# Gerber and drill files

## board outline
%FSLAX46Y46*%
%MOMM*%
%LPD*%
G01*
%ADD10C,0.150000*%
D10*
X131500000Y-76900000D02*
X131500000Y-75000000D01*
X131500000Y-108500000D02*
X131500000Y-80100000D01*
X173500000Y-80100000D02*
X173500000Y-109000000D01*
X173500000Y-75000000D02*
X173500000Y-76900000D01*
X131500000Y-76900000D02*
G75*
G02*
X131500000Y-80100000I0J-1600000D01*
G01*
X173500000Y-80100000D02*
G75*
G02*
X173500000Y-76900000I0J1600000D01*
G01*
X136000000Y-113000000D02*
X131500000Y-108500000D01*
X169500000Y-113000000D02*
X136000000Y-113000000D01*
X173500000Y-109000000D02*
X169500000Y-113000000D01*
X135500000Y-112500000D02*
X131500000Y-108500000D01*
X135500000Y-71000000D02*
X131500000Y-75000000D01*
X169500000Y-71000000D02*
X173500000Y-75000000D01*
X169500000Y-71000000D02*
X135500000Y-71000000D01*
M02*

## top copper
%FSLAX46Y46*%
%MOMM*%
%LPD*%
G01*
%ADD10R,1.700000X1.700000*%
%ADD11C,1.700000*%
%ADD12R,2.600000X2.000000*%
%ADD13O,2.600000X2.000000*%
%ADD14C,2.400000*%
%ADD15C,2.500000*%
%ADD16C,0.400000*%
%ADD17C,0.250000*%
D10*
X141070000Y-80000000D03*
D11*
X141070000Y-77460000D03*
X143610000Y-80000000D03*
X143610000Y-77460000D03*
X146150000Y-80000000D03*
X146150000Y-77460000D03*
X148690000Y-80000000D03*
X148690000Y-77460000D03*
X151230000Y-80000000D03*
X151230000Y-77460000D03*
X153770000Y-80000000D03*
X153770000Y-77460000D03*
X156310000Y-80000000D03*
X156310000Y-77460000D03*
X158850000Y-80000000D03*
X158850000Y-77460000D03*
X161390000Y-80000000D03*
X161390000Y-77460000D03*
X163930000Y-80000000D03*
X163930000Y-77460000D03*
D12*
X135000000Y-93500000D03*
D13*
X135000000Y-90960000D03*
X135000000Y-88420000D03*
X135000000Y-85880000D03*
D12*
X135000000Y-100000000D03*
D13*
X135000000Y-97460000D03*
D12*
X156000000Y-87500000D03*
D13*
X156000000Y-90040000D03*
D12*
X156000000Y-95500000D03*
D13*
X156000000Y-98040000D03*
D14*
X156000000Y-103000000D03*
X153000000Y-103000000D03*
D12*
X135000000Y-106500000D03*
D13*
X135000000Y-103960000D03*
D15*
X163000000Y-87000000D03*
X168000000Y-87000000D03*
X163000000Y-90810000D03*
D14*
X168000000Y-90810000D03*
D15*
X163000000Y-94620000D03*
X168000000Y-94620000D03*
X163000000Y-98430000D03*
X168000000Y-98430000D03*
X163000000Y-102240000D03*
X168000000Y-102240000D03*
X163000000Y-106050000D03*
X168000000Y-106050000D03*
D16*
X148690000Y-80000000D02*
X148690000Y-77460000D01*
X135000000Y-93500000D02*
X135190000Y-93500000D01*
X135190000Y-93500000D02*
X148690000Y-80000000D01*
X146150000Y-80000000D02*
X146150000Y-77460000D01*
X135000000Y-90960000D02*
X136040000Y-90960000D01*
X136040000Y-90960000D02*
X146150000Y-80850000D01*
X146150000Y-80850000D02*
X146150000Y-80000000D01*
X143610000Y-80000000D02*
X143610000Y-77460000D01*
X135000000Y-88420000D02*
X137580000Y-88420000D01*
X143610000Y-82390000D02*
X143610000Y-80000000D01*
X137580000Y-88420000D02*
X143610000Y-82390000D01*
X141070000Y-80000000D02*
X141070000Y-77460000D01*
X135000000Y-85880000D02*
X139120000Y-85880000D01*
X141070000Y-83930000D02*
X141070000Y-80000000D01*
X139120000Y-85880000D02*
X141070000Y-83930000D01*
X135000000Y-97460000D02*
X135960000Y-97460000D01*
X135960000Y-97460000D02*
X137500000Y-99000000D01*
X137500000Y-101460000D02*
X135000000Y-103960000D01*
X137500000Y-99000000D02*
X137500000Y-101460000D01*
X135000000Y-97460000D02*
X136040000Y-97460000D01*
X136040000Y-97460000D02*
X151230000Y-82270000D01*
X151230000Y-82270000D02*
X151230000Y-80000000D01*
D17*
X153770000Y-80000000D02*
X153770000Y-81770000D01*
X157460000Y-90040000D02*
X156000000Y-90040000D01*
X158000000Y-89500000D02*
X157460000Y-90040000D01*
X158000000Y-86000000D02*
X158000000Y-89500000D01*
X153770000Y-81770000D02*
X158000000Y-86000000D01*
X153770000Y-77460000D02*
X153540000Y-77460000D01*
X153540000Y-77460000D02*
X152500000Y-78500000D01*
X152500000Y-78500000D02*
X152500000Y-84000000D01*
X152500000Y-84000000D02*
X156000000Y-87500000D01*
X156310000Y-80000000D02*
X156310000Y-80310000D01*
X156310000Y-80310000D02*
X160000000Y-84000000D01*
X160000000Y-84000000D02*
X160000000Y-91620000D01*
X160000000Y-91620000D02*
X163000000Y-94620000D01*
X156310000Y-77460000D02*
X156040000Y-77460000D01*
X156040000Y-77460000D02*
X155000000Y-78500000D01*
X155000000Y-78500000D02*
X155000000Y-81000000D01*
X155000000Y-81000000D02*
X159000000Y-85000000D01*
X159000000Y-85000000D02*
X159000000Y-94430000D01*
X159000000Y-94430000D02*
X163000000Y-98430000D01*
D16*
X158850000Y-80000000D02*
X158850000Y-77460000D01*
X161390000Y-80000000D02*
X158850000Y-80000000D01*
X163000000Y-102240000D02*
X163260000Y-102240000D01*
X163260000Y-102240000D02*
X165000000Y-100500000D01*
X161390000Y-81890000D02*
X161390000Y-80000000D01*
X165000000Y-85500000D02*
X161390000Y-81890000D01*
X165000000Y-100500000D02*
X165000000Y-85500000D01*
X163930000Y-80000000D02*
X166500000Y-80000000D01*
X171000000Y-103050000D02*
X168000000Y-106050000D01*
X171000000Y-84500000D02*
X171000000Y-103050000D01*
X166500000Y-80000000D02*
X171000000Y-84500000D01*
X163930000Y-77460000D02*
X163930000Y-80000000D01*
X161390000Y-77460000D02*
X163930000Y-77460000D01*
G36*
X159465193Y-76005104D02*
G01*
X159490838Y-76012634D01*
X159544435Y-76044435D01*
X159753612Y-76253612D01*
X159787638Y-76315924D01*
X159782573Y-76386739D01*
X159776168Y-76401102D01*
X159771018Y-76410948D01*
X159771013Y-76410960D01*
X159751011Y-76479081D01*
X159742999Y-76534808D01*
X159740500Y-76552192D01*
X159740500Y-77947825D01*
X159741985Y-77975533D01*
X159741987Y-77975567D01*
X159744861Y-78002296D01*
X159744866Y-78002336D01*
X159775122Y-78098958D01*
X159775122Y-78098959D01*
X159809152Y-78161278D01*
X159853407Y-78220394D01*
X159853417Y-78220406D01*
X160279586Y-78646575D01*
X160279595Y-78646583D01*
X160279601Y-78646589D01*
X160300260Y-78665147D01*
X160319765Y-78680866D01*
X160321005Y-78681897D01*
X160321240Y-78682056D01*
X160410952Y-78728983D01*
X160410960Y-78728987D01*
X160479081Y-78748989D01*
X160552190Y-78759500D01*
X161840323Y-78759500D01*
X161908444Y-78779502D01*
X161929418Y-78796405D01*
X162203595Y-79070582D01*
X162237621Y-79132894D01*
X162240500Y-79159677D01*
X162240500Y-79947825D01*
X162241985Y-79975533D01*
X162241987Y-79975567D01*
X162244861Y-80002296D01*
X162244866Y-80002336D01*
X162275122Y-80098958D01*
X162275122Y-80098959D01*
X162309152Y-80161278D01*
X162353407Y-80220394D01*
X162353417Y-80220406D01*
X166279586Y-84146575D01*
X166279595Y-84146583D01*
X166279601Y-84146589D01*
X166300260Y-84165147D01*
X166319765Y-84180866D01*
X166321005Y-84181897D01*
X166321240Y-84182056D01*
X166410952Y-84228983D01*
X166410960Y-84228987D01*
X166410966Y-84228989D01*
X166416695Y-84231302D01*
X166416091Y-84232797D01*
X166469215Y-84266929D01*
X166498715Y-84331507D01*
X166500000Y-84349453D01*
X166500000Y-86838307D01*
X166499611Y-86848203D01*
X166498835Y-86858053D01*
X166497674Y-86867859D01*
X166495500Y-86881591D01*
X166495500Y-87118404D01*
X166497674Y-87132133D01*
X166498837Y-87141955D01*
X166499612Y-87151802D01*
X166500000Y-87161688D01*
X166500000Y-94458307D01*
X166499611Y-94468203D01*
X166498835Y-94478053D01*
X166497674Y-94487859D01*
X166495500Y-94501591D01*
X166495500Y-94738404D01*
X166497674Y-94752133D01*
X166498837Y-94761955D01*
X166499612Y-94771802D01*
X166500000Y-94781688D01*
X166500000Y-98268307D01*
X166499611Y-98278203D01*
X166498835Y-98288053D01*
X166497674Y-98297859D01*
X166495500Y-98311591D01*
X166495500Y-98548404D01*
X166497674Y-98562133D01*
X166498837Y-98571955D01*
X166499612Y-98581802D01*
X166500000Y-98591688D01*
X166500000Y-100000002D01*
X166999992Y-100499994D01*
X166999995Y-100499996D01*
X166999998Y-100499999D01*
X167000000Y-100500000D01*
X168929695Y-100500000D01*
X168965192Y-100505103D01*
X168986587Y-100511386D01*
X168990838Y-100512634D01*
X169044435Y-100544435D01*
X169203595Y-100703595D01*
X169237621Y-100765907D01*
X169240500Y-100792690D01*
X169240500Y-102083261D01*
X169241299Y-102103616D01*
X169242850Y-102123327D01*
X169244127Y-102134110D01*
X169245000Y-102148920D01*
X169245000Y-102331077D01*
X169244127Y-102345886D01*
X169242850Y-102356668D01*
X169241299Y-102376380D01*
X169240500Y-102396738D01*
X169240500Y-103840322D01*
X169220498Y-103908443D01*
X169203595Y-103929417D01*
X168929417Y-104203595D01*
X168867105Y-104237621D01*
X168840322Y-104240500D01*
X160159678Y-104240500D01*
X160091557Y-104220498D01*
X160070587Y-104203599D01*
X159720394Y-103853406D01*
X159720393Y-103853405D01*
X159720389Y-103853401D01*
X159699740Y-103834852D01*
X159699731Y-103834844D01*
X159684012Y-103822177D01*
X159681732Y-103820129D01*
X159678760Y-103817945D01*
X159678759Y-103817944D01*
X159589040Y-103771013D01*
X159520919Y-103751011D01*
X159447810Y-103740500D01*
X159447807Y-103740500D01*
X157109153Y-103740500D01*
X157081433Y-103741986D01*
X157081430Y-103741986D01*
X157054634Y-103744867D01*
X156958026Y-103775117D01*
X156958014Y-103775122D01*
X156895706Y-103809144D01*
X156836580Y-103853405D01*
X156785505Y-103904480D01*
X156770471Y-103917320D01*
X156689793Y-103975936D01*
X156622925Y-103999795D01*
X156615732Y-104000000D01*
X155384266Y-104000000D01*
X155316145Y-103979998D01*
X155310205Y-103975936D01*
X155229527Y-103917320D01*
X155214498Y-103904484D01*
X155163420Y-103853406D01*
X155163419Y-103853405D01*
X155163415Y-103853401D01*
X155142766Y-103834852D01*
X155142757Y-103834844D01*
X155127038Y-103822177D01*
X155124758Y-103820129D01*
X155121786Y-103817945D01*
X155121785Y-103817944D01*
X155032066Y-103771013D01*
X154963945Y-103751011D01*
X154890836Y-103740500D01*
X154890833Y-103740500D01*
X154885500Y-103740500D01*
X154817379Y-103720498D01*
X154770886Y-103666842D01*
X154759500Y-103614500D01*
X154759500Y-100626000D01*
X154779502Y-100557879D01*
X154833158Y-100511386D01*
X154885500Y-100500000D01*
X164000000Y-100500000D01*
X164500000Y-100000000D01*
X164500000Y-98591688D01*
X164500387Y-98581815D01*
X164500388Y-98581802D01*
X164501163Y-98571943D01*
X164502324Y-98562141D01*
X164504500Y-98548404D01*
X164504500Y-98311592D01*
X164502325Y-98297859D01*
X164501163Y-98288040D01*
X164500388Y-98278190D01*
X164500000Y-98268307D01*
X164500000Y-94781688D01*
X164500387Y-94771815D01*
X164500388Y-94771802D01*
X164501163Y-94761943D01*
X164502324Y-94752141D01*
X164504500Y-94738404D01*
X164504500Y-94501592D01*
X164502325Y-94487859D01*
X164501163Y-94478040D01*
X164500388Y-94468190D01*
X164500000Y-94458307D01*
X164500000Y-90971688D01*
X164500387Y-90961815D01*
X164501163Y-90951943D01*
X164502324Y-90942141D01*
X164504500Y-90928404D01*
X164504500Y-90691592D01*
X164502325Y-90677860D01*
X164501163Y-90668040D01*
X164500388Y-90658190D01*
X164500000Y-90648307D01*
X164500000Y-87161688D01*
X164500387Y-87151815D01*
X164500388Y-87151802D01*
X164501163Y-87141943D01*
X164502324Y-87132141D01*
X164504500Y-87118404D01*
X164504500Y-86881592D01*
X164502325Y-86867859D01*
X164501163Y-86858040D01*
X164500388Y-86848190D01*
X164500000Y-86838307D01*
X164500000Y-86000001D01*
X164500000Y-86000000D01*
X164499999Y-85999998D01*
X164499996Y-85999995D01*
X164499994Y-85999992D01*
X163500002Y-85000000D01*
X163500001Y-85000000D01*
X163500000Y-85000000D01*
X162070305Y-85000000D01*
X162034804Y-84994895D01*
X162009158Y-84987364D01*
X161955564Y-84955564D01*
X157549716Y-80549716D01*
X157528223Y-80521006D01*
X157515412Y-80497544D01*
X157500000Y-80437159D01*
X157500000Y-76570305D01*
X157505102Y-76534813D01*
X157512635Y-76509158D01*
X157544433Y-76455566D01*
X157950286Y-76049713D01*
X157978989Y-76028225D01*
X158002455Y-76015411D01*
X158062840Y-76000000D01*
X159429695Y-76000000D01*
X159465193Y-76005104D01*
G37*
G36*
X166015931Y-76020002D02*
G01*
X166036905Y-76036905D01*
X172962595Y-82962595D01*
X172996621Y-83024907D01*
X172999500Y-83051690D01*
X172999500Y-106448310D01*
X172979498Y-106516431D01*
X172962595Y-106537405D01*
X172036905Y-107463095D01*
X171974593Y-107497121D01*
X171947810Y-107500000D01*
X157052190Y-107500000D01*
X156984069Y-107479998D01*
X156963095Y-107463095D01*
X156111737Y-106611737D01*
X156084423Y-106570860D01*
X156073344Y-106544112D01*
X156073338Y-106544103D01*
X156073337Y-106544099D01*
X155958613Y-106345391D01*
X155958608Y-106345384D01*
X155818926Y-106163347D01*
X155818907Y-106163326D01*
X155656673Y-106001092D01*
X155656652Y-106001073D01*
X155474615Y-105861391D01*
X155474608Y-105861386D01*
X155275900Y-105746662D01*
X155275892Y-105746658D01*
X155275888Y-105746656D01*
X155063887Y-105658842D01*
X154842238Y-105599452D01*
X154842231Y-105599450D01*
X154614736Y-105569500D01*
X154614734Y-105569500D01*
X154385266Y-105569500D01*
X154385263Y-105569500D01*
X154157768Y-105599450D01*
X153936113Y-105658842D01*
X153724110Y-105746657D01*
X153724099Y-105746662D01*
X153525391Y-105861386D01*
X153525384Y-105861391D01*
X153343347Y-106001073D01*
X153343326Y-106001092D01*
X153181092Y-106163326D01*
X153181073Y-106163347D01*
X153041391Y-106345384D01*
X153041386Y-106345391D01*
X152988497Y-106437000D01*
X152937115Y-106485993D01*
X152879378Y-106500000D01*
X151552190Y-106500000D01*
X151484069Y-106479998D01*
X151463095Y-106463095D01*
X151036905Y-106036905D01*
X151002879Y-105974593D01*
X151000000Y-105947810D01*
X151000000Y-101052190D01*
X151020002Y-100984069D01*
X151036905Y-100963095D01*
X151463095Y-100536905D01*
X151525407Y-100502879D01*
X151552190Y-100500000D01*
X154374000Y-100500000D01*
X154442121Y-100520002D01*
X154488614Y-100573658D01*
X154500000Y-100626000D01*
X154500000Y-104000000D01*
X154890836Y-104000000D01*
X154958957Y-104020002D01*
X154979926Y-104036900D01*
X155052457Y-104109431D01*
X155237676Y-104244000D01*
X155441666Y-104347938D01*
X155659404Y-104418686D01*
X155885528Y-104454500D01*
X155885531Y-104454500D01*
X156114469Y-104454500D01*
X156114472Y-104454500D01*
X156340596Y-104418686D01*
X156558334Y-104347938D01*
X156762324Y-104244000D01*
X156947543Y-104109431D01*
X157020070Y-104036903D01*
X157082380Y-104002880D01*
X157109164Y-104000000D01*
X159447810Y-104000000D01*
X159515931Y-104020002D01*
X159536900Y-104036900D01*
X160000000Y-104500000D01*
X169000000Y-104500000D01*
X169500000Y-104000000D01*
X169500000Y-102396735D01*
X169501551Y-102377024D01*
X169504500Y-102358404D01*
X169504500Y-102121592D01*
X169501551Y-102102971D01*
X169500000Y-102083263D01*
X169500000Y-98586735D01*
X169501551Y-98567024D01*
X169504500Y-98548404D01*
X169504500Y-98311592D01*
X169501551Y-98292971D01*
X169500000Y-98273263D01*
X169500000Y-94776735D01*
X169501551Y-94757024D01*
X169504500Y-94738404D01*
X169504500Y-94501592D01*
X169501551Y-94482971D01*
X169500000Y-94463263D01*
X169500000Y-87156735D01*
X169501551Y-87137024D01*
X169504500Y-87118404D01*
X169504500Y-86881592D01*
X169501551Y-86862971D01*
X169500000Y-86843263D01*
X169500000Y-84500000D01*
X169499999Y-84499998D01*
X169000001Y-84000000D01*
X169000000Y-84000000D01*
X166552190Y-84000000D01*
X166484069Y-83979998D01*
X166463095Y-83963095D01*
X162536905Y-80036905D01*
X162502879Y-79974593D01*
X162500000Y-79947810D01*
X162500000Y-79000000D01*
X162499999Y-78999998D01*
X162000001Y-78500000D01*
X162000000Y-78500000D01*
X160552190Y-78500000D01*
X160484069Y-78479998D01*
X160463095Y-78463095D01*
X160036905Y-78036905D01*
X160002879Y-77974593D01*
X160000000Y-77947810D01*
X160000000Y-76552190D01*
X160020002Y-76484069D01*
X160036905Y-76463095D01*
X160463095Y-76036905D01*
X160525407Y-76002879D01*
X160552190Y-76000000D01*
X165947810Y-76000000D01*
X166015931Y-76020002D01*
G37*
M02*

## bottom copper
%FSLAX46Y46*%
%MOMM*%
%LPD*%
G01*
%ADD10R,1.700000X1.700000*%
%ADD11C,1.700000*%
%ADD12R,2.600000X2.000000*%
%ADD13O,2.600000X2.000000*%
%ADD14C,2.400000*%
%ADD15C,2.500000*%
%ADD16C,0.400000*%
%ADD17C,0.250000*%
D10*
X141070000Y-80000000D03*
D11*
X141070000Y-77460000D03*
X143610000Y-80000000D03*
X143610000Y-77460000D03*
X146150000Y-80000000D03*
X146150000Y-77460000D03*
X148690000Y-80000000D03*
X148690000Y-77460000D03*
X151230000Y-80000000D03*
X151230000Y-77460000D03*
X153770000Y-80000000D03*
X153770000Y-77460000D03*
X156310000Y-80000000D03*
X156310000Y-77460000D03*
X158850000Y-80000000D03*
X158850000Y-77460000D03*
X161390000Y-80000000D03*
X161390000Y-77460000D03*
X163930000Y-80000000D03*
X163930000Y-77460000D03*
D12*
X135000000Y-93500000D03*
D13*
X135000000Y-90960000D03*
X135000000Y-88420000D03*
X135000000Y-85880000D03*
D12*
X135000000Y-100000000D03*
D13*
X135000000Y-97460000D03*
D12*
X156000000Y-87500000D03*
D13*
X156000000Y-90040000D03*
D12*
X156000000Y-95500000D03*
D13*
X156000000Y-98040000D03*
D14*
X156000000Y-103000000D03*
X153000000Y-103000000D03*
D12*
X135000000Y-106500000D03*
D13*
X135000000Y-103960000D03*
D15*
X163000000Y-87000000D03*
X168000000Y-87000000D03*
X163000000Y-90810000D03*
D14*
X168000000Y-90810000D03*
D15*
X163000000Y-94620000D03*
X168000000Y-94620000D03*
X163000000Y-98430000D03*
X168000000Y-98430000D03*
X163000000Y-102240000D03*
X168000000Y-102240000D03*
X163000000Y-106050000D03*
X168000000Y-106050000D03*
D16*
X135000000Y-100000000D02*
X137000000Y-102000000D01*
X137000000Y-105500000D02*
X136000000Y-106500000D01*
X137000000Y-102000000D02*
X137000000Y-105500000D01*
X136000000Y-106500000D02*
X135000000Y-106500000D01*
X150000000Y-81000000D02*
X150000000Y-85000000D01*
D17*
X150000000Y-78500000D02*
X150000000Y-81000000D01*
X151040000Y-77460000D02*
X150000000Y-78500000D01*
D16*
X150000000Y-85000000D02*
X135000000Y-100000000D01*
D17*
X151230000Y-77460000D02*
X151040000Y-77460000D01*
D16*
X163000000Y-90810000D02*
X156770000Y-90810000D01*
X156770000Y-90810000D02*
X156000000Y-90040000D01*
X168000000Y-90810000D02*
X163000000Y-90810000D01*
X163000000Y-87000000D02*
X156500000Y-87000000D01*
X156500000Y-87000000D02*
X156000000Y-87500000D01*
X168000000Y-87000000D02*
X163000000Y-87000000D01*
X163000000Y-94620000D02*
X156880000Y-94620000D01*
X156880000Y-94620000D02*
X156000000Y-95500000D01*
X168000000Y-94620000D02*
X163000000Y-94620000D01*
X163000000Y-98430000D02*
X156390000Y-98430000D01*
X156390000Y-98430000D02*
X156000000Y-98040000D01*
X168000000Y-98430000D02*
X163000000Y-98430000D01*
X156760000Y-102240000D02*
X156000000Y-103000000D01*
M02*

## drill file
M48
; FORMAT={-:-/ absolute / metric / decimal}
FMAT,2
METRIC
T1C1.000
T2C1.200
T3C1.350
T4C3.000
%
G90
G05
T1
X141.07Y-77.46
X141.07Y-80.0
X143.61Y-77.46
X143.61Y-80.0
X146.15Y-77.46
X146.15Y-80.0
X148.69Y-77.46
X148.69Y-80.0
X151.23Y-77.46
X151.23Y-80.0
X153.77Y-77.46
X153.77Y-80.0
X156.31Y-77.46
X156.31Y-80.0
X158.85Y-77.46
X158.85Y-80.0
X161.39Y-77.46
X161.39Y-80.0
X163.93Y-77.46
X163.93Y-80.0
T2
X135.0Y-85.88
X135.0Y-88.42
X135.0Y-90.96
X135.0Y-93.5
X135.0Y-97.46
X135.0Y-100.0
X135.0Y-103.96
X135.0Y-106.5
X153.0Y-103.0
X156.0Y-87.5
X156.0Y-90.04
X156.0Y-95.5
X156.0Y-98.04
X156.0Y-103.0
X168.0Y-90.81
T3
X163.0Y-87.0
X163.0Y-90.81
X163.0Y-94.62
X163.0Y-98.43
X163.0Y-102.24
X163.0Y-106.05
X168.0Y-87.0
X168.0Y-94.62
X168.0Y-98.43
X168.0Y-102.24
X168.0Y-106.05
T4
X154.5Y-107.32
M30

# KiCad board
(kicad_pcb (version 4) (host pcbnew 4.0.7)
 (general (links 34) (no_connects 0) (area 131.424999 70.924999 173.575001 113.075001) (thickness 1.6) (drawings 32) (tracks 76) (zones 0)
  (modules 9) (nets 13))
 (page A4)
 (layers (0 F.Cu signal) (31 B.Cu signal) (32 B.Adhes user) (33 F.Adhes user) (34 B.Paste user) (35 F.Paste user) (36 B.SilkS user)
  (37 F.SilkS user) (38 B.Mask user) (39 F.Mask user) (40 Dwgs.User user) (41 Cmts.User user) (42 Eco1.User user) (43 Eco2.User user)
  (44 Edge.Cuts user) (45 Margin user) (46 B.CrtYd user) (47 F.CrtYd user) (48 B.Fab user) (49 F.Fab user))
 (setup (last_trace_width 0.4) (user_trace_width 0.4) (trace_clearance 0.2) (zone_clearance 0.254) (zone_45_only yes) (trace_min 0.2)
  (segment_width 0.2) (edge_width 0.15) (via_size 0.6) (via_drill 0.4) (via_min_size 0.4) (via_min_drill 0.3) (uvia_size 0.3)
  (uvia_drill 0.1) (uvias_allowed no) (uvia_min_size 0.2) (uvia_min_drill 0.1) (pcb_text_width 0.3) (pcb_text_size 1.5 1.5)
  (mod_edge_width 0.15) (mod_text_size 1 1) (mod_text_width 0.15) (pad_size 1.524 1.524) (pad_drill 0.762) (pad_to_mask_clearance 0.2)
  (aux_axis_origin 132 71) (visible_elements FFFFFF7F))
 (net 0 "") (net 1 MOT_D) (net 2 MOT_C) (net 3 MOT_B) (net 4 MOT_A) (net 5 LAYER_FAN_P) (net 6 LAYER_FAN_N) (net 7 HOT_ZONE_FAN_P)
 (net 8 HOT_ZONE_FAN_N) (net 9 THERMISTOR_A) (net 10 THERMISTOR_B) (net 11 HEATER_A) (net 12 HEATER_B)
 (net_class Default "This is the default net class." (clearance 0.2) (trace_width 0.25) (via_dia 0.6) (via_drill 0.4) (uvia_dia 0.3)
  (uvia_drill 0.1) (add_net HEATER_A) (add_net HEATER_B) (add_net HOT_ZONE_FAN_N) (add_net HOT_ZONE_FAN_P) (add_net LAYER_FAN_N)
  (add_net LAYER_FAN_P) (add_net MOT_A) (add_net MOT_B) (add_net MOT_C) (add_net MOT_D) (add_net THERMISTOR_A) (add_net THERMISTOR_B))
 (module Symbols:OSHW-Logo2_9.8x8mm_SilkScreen (layer B.Cu) (at 142.5 86 90)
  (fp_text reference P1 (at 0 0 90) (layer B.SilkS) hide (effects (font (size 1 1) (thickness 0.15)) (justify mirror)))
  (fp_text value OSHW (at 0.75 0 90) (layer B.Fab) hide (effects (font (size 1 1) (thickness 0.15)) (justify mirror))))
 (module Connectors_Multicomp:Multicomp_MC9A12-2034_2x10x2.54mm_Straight (layer F.Cu) (at 141.07 80)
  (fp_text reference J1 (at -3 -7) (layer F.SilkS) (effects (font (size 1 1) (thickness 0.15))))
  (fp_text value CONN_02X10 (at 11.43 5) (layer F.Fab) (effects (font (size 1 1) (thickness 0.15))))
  (pad 1 thru_hole rect (at 0 0) (size 1.7 1.7) (drill 1) (layers *.Cu *.Mask) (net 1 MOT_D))
  (pad 2 thru_hole circle (at 0 -2.54) (size 1.7 1.7) (drill 1) (layers *.Cu *.Mask) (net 1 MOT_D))
  (pad 3 thru_hole circle (at 2.54 0) (size 1.7 1.7) (drill 1) (layers *.Cu *.Mask) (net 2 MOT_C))
  (pad 4 thru_hole circle (at 2.54 -2.54) (size 1.7 1.7) (drill 1) (layers *.Cu *.Mask) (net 2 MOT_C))
  (pad 5 thru_hole circle (at 5.08 0) (size 1.7 1.7) (drill 1) (layers *.Cu *.Mask) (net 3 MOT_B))
  (pad 6 thru_hole circle (at 5.08 -2.54) (size 1.7 1.7) (drill 1) (layers *.Cu *.Mask) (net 3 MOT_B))
  (pad 7 thru_hole circle (at 7.62 0) (size 1.7 1.7) (drill 1) (layers *.Cu *.Mask) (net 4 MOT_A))
  (pad 8 thru_hole circle (at 7.62 -2.54) (size 1.7 1.7) (drill 1) (layers *.Cu *.Mask) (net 4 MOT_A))
  (pad 9 thru_hole circle (at 10.16 0) (size 1.7 1.7) (drill 1) (layers *.Cu *.Mask) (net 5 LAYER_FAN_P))
  (pad 10 thru_hole circle (at 10.16 -2.54) (size 1.7 1.7) (drill 1) (layers *.Cu *.Mask) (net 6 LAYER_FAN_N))
  (pad 11 thru_hole circle (at 12.7 0) (size 1.7 1.7) (drill 1) (layers *.Cu *.Mask) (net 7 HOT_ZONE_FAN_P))
  (pad 12 thru_hole circle (at 12.7 -2.54) (size 1.7 1.7) (drill 1) (layers *.Cu *.Mask) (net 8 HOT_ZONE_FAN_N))
  (pad 13 thru_hole circle (at 15.24 0) (size 1.7 1.7) (drill 1) (layers *.Cu *.Mask) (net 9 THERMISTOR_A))
  (pad 14 thru_hole circle (at 15.24 -2.54) (size 1.7 1.7) (drill 1) (layers *.Cu *.Mask) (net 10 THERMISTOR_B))
  (pad 15 thru_hole circle (at 17.78 0) (size 1.7 1.7) (drill 1) (layers *.Cu *.Mask) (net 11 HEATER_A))
  (pad 16 thru_hole circle (at 17.78 -2.54) (size 1.7 1.7) (drill 1) (layers *.Cu *.Mask) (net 11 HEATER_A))
  (pad 17 thru_hole circle (at 20.32 0) (size 1.7 1.7) (drill 1) (layers *.Cu *.Mask) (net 11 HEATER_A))
  (pad 18 thru_hole circle (at 20.32 -2.54) (size 1.7 1.7) (drill 1) (layers *.Cu *.Mask) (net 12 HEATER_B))
  (pad 19 thru_hole circle (at 22.86 0) (size 1.7 1.7) (drill 1) (layers *.Cu *.Mask) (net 12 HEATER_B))
  (pad 20 thru_hole circle (at 22.86 -2.54) (size 1.7 1.7) (drill 1) (layers *.Cu *.Mask) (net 12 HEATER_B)))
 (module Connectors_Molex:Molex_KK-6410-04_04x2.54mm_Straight (layer F.Cu) (at 135 93.5 90)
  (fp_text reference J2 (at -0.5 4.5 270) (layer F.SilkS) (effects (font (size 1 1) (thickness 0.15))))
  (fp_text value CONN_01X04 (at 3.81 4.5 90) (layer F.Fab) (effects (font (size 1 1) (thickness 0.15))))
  (pad 1 thru_hole rect (at 0 0 90) (size 2 2.6) (drill 1.2) (layers *.Cu *.Mask) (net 4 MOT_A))
  (pad 2 thru_hole oval (at 2.54 0 90) (size 2 2.6) (drill 1.2) (layers *.Cu *.Mask) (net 3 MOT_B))
  (pad 3 thru_hole oval (at 5.08 0 90) (size 2 2.6) (drill 1.2) (layers *.Cu *.Mask) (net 2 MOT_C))
  (pad 4 thru_hole oval (at 7.62 0 90) (size 2 2.6) (drill 1.2) (layers *.Cu *.Mask) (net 1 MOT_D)))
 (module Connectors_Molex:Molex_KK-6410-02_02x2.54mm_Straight (layer F.Cu) (at 135 100 90)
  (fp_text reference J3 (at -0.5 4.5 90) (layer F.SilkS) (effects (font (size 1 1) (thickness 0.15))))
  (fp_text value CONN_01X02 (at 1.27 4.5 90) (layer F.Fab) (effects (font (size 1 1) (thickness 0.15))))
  (pad 1 thru_hole rect (at 0 0 90) (size 2 2.6) (drill 1.2) (layers *.Cu *.Mask) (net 6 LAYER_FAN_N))
  (pad 2 thru_hole oval (at 2.54 0 90) (size 2 2.6) (drill 1.2) (layers *.Cu *.Mask) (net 5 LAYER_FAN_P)))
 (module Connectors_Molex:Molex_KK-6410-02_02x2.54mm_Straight (layer F.Cu) (at 156 87.5 270)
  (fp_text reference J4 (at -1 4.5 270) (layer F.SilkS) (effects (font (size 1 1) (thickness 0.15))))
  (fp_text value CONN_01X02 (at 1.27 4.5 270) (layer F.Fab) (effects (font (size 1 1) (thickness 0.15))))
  (pad 1 thru_hole rect (at 0 0 270) (size 2 2.6) (drill 1.2) (layers *.Cu *.Mask) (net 8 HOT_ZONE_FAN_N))
  (pad 2 thru_hole oval (at 2.54 0 270) (size 2 2.6) (drill 1.2) (layers *.Cu *.Mask) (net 7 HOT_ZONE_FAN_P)))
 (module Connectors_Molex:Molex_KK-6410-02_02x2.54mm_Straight (layer F.Cu) (at 156 95.5 270)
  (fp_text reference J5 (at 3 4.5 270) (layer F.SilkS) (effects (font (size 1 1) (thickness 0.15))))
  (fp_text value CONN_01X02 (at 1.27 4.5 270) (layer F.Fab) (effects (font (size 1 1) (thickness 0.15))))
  (pad 1 thru_hole rect (at 0 0 270) (size 2 2.6) (drill 1.2) (layers *.Cu *.Mask) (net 9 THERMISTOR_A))
  (pad 2 thru_hole oval (at 2.54 0 270) (size 2 2.6) (drill 1.2) (layers *.Cu *.Mask) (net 10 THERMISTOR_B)))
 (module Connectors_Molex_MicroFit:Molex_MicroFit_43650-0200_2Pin (layer F.Cu) (at 154.5 103)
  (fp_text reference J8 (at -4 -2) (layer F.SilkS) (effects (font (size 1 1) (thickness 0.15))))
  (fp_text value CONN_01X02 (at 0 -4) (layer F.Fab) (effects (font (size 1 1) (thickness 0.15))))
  (pad 1 thru_hole circle (at 1.5 0) (size 2.4 2.4) (drill 1.2) (layers *.Cu *.Mask) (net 11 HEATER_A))
  (pad 2 thru_hole circle (at -1.5 0) (size 2.4 2.4) (drill 1.2) (layers *.Cu *.Mask) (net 12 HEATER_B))
  (pad "" np_thru_hole circle (at 0 4.32) (size 3 3) (drill 3) (layers *.Cu *.Mask)))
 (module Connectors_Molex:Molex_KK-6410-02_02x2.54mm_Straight (layer F.Cu) (at 135 106.5 90)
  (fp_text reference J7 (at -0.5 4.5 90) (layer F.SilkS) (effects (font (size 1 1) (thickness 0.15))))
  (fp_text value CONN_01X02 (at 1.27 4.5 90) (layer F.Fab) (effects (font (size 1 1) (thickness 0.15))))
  (pad 1 thru_hole rect (at 0 0 90) (size 2 2.6) (drill 1.2) (layers *.Cu *.Mask) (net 6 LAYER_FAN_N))
  (pad 2 thru_hole oval (at 2.54 0 90) (size 2 2.6) (drill 1.2) (layers *.Cu *.Mask) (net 5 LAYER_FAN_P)))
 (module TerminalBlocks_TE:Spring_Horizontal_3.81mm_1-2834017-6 (layer F.Cu) (at 163 87 90)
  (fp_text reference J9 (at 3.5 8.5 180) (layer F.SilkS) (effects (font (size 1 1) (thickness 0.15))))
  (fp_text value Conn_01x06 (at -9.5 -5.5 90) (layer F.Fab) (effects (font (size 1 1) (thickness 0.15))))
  (pad 1 thru_hole circle (at 0 0 90) (size 2.5 2.5) (drill 1.35) (layers *.Cu *.Mask) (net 8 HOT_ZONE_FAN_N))
  (pad 1 thru_hole circle (at 0 5 90) (size 2.5 2.5) (drill 1.35) (layers *.Cu *.Mask) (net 8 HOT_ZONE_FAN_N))
  (pad 2 thru_hole circle (at -3.81 0 90) (size 2.5 2.5) (drill 1.35) (layers *.Cu *.Mask) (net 7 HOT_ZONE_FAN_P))
  (pad 2 thru_hole circle (at -3.81 5 90) (size 2.4 2.4) (drill 1.2) (layers *.Cu *.Mask) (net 7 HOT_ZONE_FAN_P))
  (pad 3 thru_hole circle (at -7.62 0 90) (size 2.5 2.5) (drill 1.35) (layers *.Cu *.Mask) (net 9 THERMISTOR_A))
  (pad 3 thru_hole circle (at -7.62 5 90) (size 2.5 2.5) (drill 1.35) (layers *.Cu *.Mask) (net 9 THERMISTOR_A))
  (pad 4 thru_hole circle (at -11.43 0 90) (size 2.5 2.5) (drill 1.35) (layers *.Cu *.Mask) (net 10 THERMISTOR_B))
  (pad 4 thru_hole circle (at -11.43 5 90) (size 2.5 2.5) (drill 1.35) (layers *.Cu *.Mask) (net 10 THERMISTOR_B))
  (pad 5 thru_hole circle (at -15.24 0 90) (size 2.5 2.5) (drill 1.35) (layers *.Cu *.Mask) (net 11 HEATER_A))
  (pad 5 thru_hole circle (at -15.24 5 90) (size 2.5 2.5) (drill 1.35) (layers *.Cu *.Mask) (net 11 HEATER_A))
  (pad 6 thru_hole circle (at -19.05 0 90) (size 2.5 2.5) (drill 1.35) (layers *.Cu *.Mask) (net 12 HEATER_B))
  (pad 6 thru_hole circle (at -19.05 5 90) (size 2.5 2.5) (drill 1.35) (layers *.Cu *.Mask) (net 12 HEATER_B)))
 (gr_line (start 131.5 76.9) (end 131.5 75) (angle 90) (layer Edge.Cuts) (width 0.15))
 (gr_line (start 131.5 108.5) (end 131.5 80.1) (angle 90) (layer Edge.Cuts) (width 0.15))
 (gr_line (start 173.5 80.1) (end 173.5 109) (angle 90) (layer Edge.Cuts) (width 0.15))
 (gr_line (start 173.5 75) (end 173.5 76.9) (angle 90) (layer Edge.Cuts) (width 0.15))
 (gr_arc (start 131.5 78.5) (end 131.5 76.9) (angle 180) (layer Edge.Cuts) (width 0.15))
 (gr_arc (start 173.5 78.5) (end 173.5 80.1) (angle 180) (layer Edge.Cuts) (width 0.15))
 (gr_line (start 136 113) (end 131.5 108.5) (angle 90) (layer Edge.Cuts) (width 0.15))
 (gr_line (start 169.5 113) (end 136 113) (angle 90) (layer Edge.Cuts) (width 0.15))
 (gr_line (start 173.5 109) (end 169.5 113) (angle 90) (layer Edge.Cuts) (width 0.15))
 (gr_line (start 135.5 112.5) (end 131.5 108.5) (angle 90) (layer Edge.Cuts) (width 0.15))
 (gr_line (start 135.5 71) (end 131.5 75) (angle 90) (layer Edge.Cuts) (width 0.15))
 (gr_line (start 169.5 71) (end 173.5 75) (angle 90) (layer Edge.Cuts) (width 0.15))
 (gr_line (start 169.5 71) (end 135.5 71) (angle 90) (layer Edge.Cuts) (width 0.15))
 (segment (start 148.69 80) (end 148.69 77.46) (width 0.4) (layer F.Cu) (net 4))
 (segment (start 135 93.5) (end 135.19 93.5) (width 0.4) (layer F.Cu) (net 4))
 (segment (start 135.19 93.5) (end 148.69 80) (width 0.4) (layer F.Cu) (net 4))
 (segment (start 146.15 80) (end 146.15 77.46) (width 0.4) (layer F.Cu) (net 3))
 (segment (start 135 90.96) (end 136.04 90.96) (width 0.4) (layer F.Cu) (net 3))
 (segment (start 136.04 90.96) (end 146.15 80.85) (width 0.4) (layer F.Cu) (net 3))
 (segment (start 146.15 80.85) (end 146.15 80) (width 0.4) (layer F.Cu) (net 3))
 (segment (start 143.61 80) (end 143.61 77.46) (width 0.4) (layer F.Cu) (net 2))
 (segment (start 135 88.42) (end 137.58 88.42) (width 0.4) (layer F.Cu) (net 2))
 (segment (start 143.61 82.39) (end 143.61 80) (width 0.4) (layer F.Cu) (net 2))
 (segment (start 137.58 88.42) (end 143.61 82.39) (width 0.4) (layer F.Cu) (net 2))
 (segment (start 141.07 80) (end 141.07 77.46) (width 0.4) (layer F.Cu) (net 1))
 (segment (start 135 85.88) (end 139.12 85.88) (width 0.4) (layer F.Cu) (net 1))
 (segment (start 141.07 83.93) (end 141.07 80) (width 0.4) (layer F.Cu) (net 1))
 (segment (start 139.12 85.88) (end 141.07 83.93) (width 0.4) (layer F.Cu) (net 1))
 (segment (start 135 97.46) (end 135.96 97.46) (width 0.4) (layer F.Cu) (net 5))
 (segment (start 135.96 97.46) (end 137.5 99) (width 0.4) (layer F.Cu) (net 5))
 (segment (start 137.5 101.46) (end 135 103.96) (width 0.4) (layer F.Cu) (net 5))
 (segment (start 137.5 99) (end 137.5 101.46) (width 0.4) (layer F.Cu) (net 5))
 (segment (start 135 97.46) (end 136.04 97.46) (width 0.4) (layer F.Cu) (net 5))
 (segment (start 136.04 97.46) (end 151.23 82.27) (width 0.4) (layer F.Cu) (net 5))
 (segment (start 151.23 82.27) (end 151.23 80) (width 0.4) (layer F.Cu) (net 5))
 (segment (start 135 100) (end 137 102) (width 0.4) (layer B.Cu) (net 6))
 (segment (start 137 105.5) (end 136 106.5) (width 0.4) (layer B.Cu) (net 6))
 (segment (start 137 102) (end 137 105.5) (width 0.4) (layer B.Cu) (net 6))
 (segment (start 136 106.5) (end 135 106.5) (width 0.4) (layer B.Cu) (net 6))
 (segment (start 150 81) (end 150 85) (width 0.4) (layer B.Cu) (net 6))
 (segment (start 150 78.5) (end 150 81) (width 0.25) (layer B.Cu) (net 6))
 (segment (start 151.04 77.46) (end 150 78.5) (width 0.25) (layer B.Cu) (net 6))
 (segment (start 150 85) (end 135 100) (width 0.4) (layer B.Cu) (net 6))
 (segment (start 151.23 77.46) (end 151.04 77.46) (width 0.25) (layer B.Cu) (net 6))
 (segment (start 153.77 80) (end 153.77 81.77) (width 0.25) (layer F.Cu) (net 7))
 (segment (start 157.46 90.04) (end 156 90.04) (width 0.25) (layer F.Cu) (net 7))
 (segment (start 158 89.5) (end 157.46 90.04) (width 0.25) (layer F.Cu) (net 7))
 (segment (start 158 86) (end 158 89.5) (width 0.25) (layer F.Cu) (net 7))
 (segment (start 153.77 81.77) (end 158 86) (width 0.25) (layer F.Cu) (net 7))
 (segment (start 163 90.81) (end 156.77 90.81) (width 0.4) (layer B.Cu) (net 7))
 (segment (start 156.77 90.81) (end 156 90.04) (width 0.4) (layer B.Cu) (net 7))
 (segment (start 168 90.81) (end 163 90.81) (width 0.4) (layer B.Cu) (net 7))
 (segment (start 153.77 77.46) (end 153.54 77.46) (width 0.25) (layer F.Cu) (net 8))
 (segment (start 153.54 77.46) (end 152.5 78.5) (width 0.25) (layer F.Cu) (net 8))
 (segment (start 152.5 78.5) (end 152.5 84) (width 0.25) (layer F.Cu) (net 8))
 (segment (start 152.5 84) (end 156 87.5) (width 0.25) (layer F.Cu) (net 8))
 (segment (start 163 87) (end 156.5 87) (width 0.4) (layer B.Cu) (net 8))
 (segment (start 156.5 87) (end 156 87.5) (width 0.4) (layer B.Cu) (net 8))
 (segment (start 168 87) (end 163 87) (width 0.4) (layer B.Cu) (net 8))
 (segment (start 156.31 80) (end 156.31 80.31) (width 0.25) (layer F.Cu) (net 9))
 (segment (start 156.31 80.31) (end 160 84) (width 0.25) (layer F.Cu) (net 9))
 (segment (start 160 84) (end 160 91.62) (width 0.25) (layer F.Cu) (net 9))
 (segment (start 160 91.62) (end 163 94.62) (width 0.25) (layer F.Cu) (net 9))
 (segment (start 163 94.62) (end 156.88 94.62) (width 0.4) (layer B.Cu) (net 9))
 (segment (start 156.88 94.62) (end 156 95.5) (width 0.4) (layer B.Cu) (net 9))
 (segment (start 168 94.62) (end 163 94.62) (width 0.4) (layer B.Cu) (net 9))
 (segment (start 156.31 77.46) (end 156.04 77.46) (width 0.25) (layer F.Cu) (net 10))
 (segment (start 156.04 77.46) (end 155 78.5) (width 0.25) (layer F.Cu) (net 10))
 (segment (start 155 78.5) (end 155 81) (width 0.25) (layer F.Cu) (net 10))
 (segment (start 155 81) (end 159 85) (width 0.25) (layer F.Cu) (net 10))
 (segment (start 159 85) (end 159 94.43) (width 0.25) (layer F.Cu) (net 10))
 (segment (start 159 94.43) (end 163 98.43) (width 0.25) (layer F.Cu) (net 10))
 (segment (start 163 98.43) (end 156.39 98.43) (width 0.4) (layer B.Cu) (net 10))
 (segment (start 156.39 98.43) (end 156 98.04) (width 0.4) (layer B.Cu) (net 10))
 (segment (start 168 98.43) (end 163 98.43) (width 0.4) (layer B.Cu) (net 10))
 (segment (start 158.85 80) (end 158.85 77.46) (width 0.4) (layer F.Cu) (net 11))
 (segment (start 161.39 80) (end 158.85 80) (width 0.4) (layer F.Cu) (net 11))
 (segment (start 163 102.24) (end 163.26 102.24) (width 0.4) (layer F.Cu) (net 11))
 (segment (start 163.26 102.24) (end 165 100.5) (width 0.4) (layer F.Cu) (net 11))
 (segment (start 161.39 81.89) (end 161.39 80) (width 0.4) (layer F.Cu) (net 11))
 (segment (start 165 85.5) (end 161.39 81.89) (width 0.4) (layer F.Cu) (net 11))
 (segment (start 165 100.5) (end 165 85.5) (width 0.4) (layer F.Cu) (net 11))
 (segment (start 156.76 102.24) (end 156 103) (width 0.4) (layer B.Cu) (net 11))
 (segment (start 163.93 80) (end 166.5 80) (width 0.4) (layer F.Cu) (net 12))
 (segment (start 171 103.05) (end 168 106.05) (width 0.4) (layer F.Cu) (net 12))
 (segment (start 171 84.5) (end 171 103.05) (width 0.4) (layer F.Cu) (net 12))
 (segment (start 166.5 80) (end 171 84.5) (width 0.4) (layer F.Cu) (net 12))
 (segment (start 163.93 77.46) (end 163.93 80) (width 0.4) (layer F.Cu) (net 12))
 (segment (start 161.39 77.46) (end 163.93 77.46) (width 0.4) (layer F.Cu) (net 12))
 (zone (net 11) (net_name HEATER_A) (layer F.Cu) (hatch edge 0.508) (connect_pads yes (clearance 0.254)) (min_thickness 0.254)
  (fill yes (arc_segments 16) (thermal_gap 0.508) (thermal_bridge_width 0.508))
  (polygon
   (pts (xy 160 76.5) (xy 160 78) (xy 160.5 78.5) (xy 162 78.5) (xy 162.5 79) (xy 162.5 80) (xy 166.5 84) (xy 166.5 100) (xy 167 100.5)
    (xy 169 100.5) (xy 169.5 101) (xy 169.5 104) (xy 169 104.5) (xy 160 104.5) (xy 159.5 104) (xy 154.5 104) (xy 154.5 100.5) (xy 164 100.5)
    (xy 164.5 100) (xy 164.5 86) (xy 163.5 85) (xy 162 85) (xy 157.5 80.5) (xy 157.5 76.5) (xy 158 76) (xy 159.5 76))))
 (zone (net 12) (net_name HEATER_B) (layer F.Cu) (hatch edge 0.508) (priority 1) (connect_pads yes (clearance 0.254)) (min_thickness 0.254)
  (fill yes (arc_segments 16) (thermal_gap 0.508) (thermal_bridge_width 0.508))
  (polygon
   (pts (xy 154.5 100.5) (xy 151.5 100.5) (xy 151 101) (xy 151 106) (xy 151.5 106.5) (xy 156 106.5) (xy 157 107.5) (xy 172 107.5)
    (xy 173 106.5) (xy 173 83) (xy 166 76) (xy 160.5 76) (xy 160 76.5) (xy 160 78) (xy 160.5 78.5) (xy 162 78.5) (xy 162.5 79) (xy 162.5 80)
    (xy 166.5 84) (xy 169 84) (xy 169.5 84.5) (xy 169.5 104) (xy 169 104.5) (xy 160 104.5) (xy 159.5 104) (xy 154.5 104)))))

